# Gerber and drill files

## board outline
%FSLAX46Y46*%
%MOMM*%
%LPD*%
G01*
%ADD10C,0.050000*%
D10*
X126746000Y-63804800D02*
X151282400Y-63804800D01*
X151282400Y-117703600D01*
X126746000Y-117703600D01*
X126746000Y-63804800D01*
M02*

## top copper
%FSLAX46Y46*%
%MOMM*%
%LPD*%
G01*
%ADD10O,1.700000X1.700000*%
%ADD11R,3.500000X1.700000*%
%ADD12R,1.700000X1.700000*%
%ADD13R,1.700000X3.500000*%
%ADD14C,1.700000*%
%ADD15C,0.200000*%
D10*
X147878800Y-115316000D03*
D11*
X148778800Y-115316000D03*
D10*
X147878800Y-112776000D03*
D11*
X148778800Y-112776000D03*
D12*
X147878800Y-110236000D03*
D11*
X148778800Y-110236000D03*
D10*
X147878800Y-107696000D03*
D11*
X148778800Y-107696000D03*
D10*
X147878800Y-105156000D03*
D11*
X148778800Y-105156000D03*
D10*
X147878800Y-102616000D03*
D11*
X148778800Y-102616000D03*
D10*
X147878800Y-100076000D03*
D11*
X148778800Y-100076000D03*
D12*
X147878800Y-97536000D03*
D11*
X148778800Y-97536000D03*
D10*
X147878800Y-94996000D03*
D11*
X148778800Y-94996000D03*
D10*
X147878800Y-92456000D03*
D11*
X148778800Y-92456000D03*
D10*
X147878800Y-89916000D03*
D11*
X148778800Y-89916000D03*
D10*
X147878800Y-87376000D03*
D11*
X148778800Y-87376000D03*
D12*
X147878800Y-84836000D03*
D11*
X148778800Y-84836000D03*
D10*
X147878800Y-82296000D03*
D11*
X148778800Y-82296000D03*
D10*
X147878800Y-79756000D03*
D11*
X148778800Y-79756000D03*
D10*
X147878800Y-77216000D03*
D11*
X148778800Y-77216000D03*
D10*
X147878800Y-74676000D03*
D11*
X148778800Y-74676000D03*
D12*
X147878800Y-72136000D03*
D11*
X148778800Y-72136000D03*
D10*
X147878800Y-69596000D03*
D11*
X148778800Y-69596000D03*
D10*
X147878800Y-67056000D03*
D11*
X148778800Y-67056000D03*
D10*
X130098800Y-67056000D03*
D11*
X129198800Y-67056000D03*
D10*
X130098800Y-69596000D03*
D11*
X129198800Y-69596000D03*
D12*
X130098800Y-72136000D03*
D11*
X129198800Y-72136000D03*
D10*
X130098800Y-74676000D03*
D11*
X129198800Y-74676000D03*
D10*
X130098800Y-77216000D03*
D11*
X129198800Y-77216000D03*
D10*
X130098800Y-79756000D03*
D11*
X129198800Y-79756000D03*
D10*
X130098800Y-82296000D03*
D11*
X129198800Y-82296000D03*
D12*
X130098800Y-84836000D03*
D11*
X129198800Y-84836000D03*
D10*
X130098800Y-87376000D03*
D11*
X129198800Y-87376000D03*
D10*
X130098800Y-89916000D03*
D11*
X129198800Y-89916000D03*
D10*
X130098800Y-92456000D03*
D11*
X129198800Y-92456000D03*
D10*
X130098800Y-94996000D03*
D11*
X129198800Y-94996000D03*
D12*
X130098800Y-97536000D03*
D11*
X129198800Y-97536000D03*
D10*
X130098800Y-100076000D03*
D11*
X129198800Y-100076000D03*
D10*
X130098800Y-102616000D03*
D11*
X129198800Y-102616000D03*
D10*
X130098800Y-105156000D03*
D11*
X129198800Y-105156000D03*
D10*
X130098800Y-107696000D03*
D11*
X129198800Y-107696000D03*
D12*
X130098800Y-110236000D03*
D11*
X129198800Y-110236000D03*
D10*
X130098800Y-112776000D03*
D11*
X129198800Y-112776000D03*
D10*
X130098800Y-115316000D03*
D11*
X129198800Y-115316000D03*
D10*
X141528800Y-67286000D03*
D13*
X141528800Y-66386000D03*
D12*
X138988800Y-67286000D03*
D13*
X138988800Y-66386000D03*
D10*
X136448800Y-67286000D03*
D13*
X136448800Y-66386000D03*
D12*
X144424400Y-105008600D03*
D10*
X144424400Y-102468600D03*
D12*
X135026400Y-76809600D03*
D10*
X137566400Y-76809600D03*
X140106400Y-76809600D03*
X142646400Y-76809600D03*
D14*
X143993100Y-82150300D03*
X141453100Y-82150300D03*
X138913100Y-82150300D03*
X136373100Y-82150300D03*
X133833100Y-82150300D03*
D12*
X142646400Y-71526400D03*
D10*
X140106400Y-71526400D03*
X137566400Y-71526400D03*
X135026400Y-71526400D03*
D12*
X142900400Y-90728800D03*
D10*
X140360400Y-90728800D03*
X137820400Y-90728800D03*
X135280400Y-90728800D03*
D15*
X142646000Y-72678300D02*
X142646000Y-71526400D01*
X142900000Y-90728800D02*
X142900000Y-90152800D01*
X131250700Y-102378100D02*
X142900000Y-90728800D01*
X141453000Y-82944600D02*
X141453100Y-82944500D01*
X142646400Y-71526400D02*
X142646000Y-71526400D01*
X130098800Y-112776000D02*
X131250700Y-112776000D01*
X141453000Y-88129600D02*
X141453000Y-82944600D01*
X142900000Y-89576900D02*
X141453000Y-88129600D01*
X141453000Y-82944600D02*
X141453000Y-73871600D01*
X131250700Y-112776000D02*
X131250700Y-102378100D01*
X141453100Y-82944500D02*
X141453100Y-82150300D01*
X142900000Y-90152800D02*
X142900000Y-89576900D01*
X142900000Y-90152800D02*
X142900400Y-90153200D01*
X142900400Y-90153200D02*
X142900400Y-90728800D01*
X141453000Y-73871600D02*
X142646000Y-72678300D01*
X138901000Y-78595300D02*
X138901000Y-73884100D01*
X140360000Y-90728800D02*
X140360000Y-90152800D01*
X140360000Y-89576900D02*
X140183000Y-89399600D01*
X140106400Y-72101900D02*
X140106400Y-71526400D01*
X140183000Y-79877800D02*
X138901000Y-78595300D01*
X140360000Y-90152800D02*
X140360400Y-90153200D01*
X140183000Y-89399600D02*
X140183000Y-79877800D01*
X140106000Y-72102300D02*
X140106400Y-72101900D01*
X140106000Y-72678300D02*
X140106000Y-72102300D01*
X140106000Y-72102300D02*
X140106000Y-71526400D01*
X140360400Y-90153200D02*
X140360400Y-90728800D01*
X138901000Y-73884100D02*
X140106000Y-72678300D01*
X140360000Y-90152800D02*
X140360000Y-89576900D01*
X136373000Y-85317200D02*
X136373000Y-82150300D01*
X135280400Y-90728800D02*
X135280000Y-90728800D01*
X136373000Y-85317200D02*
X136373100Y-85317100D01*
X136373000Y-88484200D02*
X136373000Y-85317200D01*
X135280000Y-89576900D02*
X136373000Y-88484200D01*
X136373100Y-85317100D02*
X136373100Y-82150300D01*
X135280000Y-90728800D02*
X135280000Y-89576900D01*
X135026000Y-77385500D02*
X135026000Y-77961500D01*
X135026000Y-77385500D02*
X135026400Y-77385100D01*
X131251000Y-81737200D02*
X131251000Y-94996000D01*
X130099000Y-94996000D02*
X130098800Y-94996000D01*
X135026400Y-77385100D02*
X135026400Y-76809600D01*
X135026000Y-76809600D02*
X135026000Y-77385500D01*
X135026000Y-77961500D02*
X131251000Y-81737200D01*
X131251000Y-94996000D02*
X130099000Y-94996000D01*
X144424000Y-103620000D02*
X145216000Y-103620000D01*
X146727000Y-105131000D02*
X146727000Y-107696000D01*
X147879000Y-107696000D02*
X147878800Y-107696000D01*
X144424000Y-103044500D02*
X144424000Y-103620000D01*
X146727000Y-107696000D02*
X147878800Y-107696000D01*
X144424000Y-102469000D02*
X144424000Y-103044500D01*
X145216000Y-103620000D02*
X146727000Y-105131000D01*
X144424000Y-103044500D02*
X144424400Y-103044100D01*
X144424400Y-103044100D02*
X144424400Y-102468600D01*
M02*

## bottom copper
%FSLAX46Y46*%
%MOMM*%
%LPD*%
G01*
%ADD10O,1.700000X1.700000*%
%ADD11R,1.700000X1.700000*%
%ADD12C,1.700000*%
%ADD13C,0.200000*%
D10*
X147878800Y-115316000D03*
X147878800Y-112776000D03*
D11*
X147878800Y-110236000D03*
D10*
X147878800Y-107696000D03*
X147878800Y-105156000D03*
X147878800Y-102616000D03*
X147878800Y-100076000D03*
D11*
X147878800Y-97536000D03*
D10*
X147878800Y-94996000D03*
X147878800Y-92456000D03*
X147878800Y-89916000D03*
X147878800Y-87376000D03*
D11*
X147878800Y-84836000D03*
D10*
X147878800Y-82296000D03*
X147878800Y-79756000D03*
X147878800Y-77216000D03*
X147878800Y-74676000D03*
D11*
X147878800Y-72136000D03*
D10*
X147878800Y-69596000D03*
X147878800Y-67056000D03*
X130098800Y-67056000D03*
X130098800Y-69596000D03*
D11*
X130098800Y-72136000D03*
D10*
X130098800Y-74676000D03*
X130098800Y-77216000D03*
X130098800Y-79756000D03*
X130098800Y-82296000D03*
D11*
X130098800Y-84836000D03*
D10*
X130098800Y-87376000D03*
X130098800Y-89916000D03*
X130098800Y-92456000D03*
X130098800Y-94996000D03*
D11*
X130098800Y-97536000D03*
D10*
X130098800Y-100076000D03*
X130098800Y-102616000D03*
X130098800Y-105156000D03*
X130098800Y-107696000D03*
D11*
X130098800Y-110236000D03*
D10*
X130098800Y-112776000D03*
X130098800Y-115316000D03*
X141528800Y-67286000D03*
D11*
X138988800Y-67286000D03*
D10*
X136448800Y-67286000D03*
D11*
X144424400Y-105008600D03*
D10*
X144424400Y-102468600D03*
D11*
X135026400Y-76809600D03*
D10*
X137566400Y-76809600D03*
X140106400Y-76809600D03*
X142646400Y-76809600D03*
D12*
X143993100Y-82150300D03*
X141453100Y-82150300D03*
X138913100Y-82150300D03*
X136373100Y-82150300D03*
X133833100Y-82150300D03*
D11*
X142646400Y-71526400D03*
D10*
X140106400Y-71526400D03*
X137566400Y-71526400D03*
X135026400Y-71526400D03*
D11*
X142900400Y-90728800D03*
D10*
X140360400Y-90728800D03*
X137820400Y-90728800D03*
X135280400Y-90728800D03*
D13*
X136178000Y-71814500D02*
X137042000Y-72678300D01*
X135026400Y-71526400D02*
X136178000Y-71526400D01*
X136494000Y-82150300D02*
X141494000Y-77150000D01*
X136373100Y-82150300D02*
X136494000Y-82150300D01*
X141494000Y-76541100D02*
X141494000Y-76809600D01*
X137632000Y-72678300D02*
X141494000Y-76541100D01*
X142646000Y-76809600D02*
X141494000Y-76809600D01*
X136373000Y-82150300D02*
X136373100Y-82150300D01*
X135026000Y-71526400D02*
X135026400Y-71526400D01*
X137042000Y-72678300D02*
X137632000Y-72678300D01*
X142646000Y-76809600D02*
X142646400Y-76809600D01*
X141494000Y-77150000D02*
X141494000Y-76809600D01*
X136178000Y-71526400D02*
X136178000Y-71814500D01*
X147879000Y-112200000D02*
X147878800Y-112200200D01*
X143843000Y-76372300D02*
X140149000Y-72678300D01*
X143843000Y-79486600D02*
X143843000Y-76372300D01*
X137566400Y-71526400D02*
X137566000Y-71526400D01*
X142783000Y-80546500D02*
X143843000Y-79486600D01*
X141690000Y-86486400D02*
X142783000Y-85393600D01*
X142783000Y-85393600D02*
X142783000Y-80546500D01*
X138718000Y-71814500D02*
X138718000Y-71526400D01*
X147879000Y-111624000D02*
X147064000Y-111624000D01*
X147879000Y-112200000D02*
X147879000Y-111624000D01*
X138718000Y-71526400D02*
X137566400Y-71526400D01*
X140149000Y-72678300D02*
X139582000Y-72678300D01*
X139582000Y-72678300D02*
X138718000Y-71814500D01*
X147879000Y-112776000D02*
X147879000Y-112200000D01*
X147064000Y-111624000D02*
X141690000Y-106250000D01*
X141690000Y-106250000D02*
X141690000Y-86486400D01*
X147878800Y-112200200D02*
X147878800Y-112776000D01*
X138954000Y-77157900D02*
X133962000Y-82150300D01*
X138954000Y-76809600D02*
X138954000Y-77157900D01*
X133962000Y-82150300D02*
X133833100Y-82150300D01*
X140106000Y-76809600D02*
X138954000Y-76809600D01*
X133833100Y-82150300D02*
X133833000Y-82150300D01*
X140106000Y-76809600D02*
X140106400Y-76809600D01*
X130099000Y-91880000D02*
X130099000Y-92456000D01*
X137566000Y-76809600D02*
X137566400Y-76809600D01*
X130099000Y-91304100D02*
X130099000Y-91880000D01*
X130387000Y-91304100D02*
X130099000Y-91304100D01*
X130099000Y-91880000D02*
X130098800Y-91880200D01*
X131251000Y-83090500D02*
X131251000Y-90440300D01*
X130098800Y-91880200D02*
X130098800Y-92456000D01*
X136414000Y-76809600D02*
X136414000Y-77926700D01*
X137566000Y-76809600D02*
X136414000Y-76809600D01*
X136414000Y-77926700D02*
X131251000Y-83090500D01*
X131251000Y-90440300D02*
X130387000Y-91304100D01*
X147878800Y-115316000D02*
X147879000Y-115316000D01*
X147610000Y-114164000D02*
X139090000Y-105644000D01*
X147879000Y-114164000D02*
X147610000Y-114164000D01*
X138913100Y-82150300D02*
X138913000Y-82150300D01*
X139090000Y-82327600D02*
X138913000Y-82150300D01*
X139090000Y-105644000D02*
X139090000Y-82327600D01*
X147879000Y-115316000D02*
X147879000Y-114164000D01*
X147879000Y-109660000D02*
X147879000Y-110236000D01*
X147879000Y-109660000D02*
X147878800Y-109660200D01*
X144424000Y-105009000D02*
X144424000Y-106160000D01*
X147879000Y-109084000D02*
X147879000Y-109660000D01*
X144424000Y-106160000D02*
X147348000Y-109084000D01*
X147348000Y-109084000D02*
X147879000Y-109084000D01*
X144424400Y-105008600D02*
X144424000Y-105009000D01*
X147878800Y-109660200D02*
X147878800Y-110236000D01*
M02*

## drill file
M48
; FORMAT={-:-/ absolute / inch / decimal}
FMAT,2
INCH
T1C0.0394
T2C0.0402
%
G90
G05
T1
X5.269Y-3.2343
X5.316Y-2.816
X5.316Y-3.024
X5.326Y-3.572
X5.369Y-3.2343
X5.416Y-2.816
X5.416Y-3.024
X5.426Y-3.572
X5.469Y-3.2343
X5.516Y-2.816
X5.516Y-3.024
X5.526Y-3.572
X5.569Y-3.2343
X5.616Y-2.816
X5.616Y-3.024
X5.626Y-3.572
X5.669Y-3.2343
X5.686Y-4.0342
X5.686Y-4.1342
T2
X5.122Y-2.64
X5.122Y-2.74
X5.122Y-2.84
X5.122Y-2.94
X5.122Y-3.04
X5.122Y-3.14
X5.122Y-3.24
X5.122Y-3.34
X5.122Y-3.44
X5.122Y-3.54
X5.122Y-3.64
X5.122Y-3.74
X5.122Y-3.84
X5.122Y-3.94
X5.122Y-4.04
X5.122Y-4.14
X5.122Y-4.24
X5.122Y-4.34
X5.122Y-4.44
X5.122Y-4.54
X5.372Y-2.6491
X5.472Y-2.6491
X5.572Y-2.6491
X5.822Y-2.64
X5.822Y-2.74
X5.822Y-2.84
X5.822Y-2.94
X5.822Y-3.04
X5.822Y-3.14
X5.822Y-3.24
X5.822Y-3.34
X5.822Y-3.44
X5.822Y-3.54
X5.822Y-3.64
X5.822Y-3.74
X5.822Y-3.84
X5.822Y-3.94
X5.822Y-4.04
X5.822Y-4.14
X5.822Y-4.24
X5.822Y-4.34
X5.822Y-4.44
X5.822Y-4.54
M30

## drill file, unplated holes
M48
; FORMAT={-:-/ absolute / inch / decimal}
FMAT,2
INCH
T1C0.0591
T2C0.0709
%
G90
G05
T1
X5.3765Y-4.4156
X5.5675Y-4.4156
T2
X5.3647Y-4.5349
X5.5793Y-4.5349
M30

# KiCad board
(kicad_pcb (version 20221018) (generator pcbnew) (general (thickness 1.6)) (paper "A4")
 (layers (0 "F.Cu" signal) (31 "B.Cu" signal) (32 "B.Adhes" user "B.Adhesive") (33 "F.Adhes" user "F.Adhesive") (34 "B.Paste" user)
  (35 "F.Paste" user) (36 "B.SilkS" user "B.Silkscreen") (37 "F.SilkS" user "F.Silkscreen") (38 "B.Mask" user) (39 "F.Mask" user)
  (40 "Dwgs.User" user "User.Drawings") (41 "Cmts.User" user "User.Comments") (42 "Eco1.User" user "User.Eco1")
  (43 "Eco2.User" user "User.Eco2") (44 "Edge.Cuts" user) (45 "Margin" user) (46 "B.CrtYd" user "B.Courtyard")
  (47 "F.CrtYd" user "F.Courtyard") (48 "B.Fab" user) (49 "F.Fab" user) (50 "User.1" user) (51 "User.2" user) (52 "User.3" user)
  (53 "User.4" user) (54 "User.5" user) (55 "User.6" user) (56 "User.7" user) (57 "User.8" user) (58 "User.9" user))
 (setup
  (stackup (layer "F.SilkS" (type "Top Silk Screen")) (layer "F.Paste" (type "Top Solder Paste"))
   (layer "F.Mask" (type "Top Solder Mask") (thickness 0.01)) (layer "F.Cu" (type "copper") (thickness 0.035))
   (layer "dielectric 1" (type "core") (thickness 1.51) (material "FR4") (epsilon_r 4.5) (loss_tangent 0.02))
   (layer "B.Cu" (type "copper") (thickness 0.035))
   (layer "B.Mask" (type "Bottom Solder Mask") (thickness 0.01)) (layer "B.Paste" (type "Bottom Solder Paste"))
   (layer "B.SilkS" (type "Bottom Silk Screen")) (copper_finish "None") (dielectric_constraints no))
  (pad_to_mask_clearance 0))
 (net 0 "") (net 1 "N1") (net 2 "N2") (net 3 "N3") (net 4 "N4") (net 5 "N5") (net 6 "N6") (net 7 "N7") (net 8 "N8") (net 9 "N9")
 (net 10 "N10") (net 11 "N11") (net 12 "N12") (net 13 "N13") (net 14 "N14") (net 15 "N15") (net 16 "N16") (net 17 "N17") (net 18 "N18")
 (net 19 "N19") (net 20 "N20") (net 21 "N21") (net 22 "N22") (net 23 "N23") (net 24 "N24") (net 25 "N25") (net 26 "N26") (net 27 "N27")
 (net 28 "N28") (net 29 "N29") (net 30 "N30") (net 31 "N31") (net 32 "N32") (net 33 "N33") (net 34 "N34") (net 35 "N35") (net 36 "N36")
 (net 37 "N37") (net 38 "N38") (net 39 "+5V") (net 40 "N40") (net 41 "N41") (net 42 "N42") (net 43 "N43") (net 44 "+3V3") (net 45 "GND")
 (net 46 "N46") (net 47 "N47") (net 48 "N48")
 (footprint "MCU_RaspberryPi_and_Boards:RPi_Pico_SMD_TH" (layer "F.Cu") (at 138.9888 91.186 180)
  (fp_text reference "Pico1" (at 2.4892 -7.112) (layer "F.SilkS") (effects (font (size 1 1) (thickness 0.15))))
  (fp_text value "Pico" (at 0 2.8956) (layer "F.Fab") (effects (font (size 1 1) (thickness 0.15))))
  (pad "" np_thru_hole oval (at -2.725 -24 180) (size 1.8 1.8) (drill 1.8) (layers "*.Cu" "*.Mask"))
  (pad "" np_thru_hole oval (at -2.425 -20.97 180) (size 1.5 1.5) (drill 1.5) (layers "*.Cu" "*.Mask"))
  (pad "" np_thru_hole oval (at 2.425 -20.97 180) (size 1.5 1.5) (drill 1.5) (layers "*.Cu" "*.Mask"))
  (pad "" np_thru_hole oval (at 2.725 -24 180) (size 1.8 1.8) (drill 1.8) (layers "*.Cu" "*.Mask"))
  (pad "1" thru_hole oval (at -8.89 -24.13 180) (size 1.7 1.7) (drill 1.02) (layers "*.Cu" "*.Mask") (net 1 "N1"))
  (pad "1" smd rect (at -8.89 -24.13 180) (size 3.5 1.7) (drill (offset -0.9 0)) (layers "F.Cu" "F.Mask") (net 1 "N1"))
  (pad "2" thru_hole oval (at -8.89 -21.59 180) (size 1.7 1.7) (drill 1.02) (layers "*.Cu" "*.Mask") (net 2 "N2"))
  (pad "2" smd rect (at -8.89 -21.59 180) (size 3.5 1.7) (drill (offset -0.9 0)) (layers "F.Cu" "F.Mask") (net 2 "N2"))
  (pad "3" thru_hole rect (at -8.89 -19.05 180) (size 1.7 1.7) (drill 1.02) (layers "*.Cu" "*.Mask") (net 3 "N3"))
  (pad "3" smd rect (at -8.89 -19.05 180) (size 3.5 1.7) (drill (offset -0.9 0)) (layers "F.Cu" "F.Mask") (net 3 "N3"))
  (pad "4" thru_hole oval (at -8.89 -16.51 180) (size 1.7 1.7) (drill 1.02) (layers "*.Cu" "*.Mask") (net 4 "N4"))
  (pad "4" smd rect (at -8.89 -16.51 180) (size 3.5 1.7) (drill (offset -0.9 0)) (layers "F.Cu" "F.Mask") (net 4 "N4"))
  (pad "5" thru_hole oval (at -8.89 -13.97 180) (size 1.7 1.7) (drill 1.02) (layers "*.Cu" "*.Mask") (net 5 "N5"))
  (pad "5" smd rect (at -8.89 -13.97 180) (size 3.5 1.7) (drill (offset -0.9 0)) (layers "F.Cu" "F.Mask") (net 5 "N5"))
  (pad "6" thru_hole oval (at -8.89 -11.43 180) (size 1.7 1.7) (drill 1.02) (layers "*.Cu" "*.Mask") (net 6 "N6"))
  (pad "6" smd rect (at -8.89 -11.43 180) (size 3.5 1.7) (drill (offset -0.9 0)) (layers "F.Cu" "F.Mask") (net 6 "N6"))
  (pad "7" thru_hole oval (at -8.89 -8.89 180) (size 1.7 1.7) (drill 1.02) (layers "*.Cu" "*.Mask") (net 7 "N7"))
  (pad "7" smd rect (at -8.89 -8.89 180) (size 3.5 1.7) (drill (offset -0.9 0)) (layers "F.Cu" "F.Mask") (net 7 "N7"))
  (pad "8" thru_hole rect (at -8.89 -6.35 180) (size 1.7 1.7) (drill 1.02) (layers "*.Cu" "*.Mask") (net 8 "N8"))
  (pad "8" smd rect (at -8.89 -6.35 180) (size 3.5 1.7) (drill (offset -0.9 0)) (layers "F.Cu" "F.Mask") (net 8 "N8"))
  (pad "9" thru_hole oval (at -8.89 -3.81 180) (size 1.7 1.7) (drill 1.02) (layers "*.Cu" "*.Mask") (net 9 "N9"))
  (pad "9" smd rect (at -8.89 -3.81 180) (size 3.5 1.7) (drill (offset -0.9 0)) (layers "F.Cu" "F.Mask") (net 9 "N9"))
  (pad "10" thru_hole oval (at -8.89 -1.27 180) (size 1.7 1.7) (drill 1.02) (layers "*.Cu" "*.Mask") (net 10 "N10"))
  (pad "10" smd rect (at -8.89 -1.27 180) (size 3.5 1.7) (drill (offset -0.9 0)) (layers "F.Cu" "F.Mask") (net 10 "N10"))
  (pad "11" thru_hole oval (at -8.89 1.27 180) (size 1.7 1.7) (drill 1.02) (layers "*.Cu" "*.Mask") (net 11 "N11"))
  (pad "11" smd rect (at -8.89 1.27 180) (size 3.5 1.7) (drill (offset -0.9 0)) (layers "F.Cu" "F.Mask") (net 11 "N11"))
  (pad "12" thru_hole oval (at -8.89 3.81 180) (size 1.7 1.7) (drill 1.02) (layers "*.Cu" "*.Mask") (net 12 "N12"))
  (pad "12" smd rect (at -8.89 3.81 180) (size 3.5 1.7) (drill (offset -0.9 0)) (layers "F.Cu" "F.Mask") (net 12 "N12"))
  (pad "13" thru_hole rect (at -8.89 6.35 180) (size 1.7 1.7) (drill 1.02) (layers "*.Cu" "*.Mask") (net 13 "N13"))
  (pad "13" smd rect (at -8.89 6.35 180) (size 3.5 1.7) (drill (offset -0.9 0)) (layers "F.Cu" "F.Mask") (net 13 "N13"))
  (pad "14" thru_hole oval (at -8.89 8.89 180) (size 1.7 1.7) (drill 1.02) (layers "*.Cu" "*.Mask") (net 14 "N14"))
  (pad "14" smd rect (at -8.89 8.89 180) (size 3.5 1.7) (drill (offset -0.9 0)) (layers "F.Cu" "F.Mask") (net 14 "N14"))
  (pad "15" thru_hole oval (at -8.89 11.43 180) (size 1.7 1.7) (drill 1.02) (layers "*.Cu" "*.Mask") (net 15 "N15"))
  (pad "15" smd rect (at -8.89 11.43 180) (size 3.5 1.7) (drill (offset -0.9 0)) (layers "F.Cu" "F.Mask") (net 15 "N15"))
  (pad "16" thru_hole oval (at -8.89 13.97 180) (size 1.7 1.7) (drill 1.02) (layers "*.Cu" "*.Mask") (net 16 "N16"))
  (pad "16" smd rect (at -8.89 13.97 180) (size 3.5 1.7) (drill (offset -0.9 0)) (layers "F.Cu" "F.Mask") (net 16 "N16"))
  (pad "17" thru_hole oval (at -8.89 16.51 180) (size 1.7 1.7) (drill 1.02) (layers "*.Cu" "*.Mask") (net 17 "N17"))
  (pad "17" smd rect (at -8.89 16.51 180) (size 3.5 1.7) (drill (offset -0.9 0)) (layers "F.Cu" "F.Mask") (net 17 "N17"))
  (pad "18" thru_hole rect (at -8.89 19.05 180) (size 1.7 1.7) (drill 1.02) (layers "*.Cu" "*.Mask") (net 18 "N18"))
  (pad "18" smd rect (at -8.89 19.05 180) (size 3.5 1.7) (drill (offset -0.9 0)) (layers "F.Cu" "F.Mask") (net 18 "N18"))
  (pad "19" thru_hole oval (at -8.89 21.59 180) (size 1.7 1.7) (drill 1.02) (layers "*.Cu" "*.Mask") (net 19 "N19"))
  (pad "19" smd rect (at -8.89 21.59 180) (size 3.5 1.7) (drill (offset -0.9 0)) (layers "F.Cu" "F.Mask") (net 19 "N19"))
  (pad "20" thru_hole oval (at -8.89 24.13 180) (size 1.7 1.7) (drill 1.02) (layers "*.Cu" "*.Mask") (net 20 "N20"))
  (pad "20" smd rect (at -8.89 24.13 180) (size 3.5 1.7) (drill (offset -0.9 0)) (layers "F.Cu" "F.Mask") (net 20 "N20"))
  (pad "21" thru_hole oval (at 8.89 24.13 180) (size 1.7 1.7) (drill 1.02) (layers "*.Cu" "*.Mask") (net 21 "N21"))
  (pad "21" smd rect (at 8.89 24.13 180) (size 3.5 1.7) (drill (offset 0.9 0)) (layers "F.Cu" "F.Mask") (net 21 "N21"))
  (pad "22" thru_hole oval (at 8.89 21.59 180) (size 1.7 1.7) (drill 1.02) (layers "*.Cu" "*.Mask") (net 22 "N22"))
  (pad "22" smd rect (at 8.89 21.59 180) (size 3.5 1.7) (drill (offset 0.9 0)) (layers "F.Cu" "F.Mask") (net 22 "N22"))
  (pad "23" thru_hole rect (at 8.89 19.05 180) (size 1.7 1.7) (drill 1.02) (layers "*.Cu" "*.Mask") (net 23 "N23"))
  (pad "23" smd rect (at 8.89 19.05 180) (size 3.5 1.7) (drill (offset 0.9 0)) (layers "F.Cu" "F.Mask") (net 23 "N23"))
  (pad "24" thru_hole oval (at 8.89 16.51 180) (size 1.7 1.7) (drill 1.02) (layers "*.Cu" "*.Mask") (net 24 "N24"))
  (pad "24" smd rect (at 8.89 16.51 180) (size 3.5 1.7) (drill (offset 0.9 0)) (layers "F.Cu" "F.Mask") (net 24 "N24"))
  (pad "25" thru_hole oval (at 8.89 13.97 180) (size 1.7 1.7) (drill 1.02) (layers "*.Cu" "*.Mask") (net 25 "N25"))
  (pad "25" smd rect (at 8.89 13.97 180) (size 3.5 1.7) (drill (offset 0.9 0)) (layers "F.Cu" "F.Mask") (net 25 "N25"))
  (pad "26" thru_hole oval (at 8.89 11.43 180) (size 1.7 1.7) (drill 1.02) (layers "*.Cu" "*.Mask") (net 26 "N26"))
  (pad "26" smd rect (at 8.89 11.43 180) (size 3.5 1.7) (drill (offset 0.9 0)) (layers "F.Cu" "F.Mask") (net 26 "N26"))
  (pad "27" thru_hole oval (at 8.89 8.89 180) (size 1.7 1.7) (drill 1.02) (layers "*.Cu" "*.Mask") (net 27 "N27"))
  (pad "27" smd rect (at 8.89 8.89 180) (size 3.5 1.7) (drill (offset 0.9 0)) (layers "F.Cu" "F.Mask") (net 27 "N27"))
  (pad "28" thru_hole rect (at 8.89 6.35 180) (size 1.7 1.7) (drill 1.02) (layers "*.Cu" "*.Mask") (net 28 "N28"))
  (pad "28" smd rect (at 8.89 6.35 180) (size 3.5 1.7) (drill (offset 0.9 0)) (layers "F.Cu" "F.Mask") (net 28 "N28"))
  (pad "29" thru_hole oval (at 8.89 3.81 180) (size 1.7 1.7) (drill 1.02) (layers "*.Cu" "*.Mask") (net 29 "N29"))
  (pad "29" smd rect (at 8.89 3.81 180) (size 3.5 1.7) (drill (offset 0.9 0)) (layers "F.Cu" "F.Mask") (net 29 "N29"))
  (pad "30" thru_hole oval (at 8.89 1.27 180) (size 1.7 1.7) (drill 1.02) (layers "*.Cu" "*.Mask") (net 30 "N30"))
  (pad "30" smd rect (at 8.89 1.27 180) (size 3.5 1.7) (drill (offset 0.9 0)) (layers "F.Cu" "F.Mask") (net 30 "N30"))
  (pad "31" thru_hole oval (at 8.89 -1.27 180) (size 1.7 1.7) (drill 1.02) (layers "*.Cu" "*.Mask") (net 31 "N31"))
  (pad "31" smd rect (at 8.89 -1.27 180) (size 3.5 1.7) (drill (offset 0.9 0)) (layers "F.Cu" "F.Mask") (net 31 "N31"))
  (pad "32" thru_hole oval (at 8.89 -3.81 180) (size 1.7 1.7) (drill 1.02) (layers "*.Cu" "*.Mask") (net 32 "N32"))
  (pad "32" smd rect (at 8.89 -3.81 180) (size 3.5 1.7) (drill (offset 0.9 0)) (layers "F.Cu" "F.Mask") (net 32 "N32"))
  (pad "33" thru_hole rect (at 8.89 -6.35 180) (size 1.7 1.7) (drill 1.02) (layers "*.Cu" "*.Mask") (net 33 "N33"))
  (pad "33" smd rect (at 8.89 -6.35 180) (size 3.5 1.7) (drill (offset 0.9 0)) (layers "F.Cu" "F.Mask") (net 33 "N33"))
  (pad "34" thru_hole oval (at 8.89 -8.89 180) (size 1.7 1.7) (drill 1.02) (layers "*.Cu" "*.Mask") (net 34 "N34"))
  (pad "34" smd rect (at 8.89 -8.89 180) (size 3.5 1.7) (drill (offset 0.9 0)) (layers "F.Cu" "F.Mask") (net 34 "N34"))
  (pad "35" thru_hole oval (at 8.89 -11.43 180) (size 1.7 1.7) (drill 1.02) (layers "*.Cu" "*.Mask") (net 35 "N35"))
  (pad "35" smd rect (at 8.89 -11.43 180) (size 3.5 1.7) (drill (offset 0.9 0)) (layers "F.Cu" "F.Mask") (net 35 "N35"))
  (pad "36" thru_hole oval (at 8.89 -13.97 180) (size 1.7 1.7) (drill 1.02) (layers "*.Cu" "*.Mask") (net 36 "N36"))
  (pad "36" smd rect (at 8.89 -13.97 180) (size 3.5 1.7) (drill (offset 0.9 0)) (layers "F.Cu" "F.Mask") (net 36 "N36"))
  (pad "37" thru_hole oval (at 8.89 -16.51 180) (size 1.7 1.7) (drill 1.02) (layers "*.Cu" "*.Mask") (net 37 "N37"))
  (pad "37" smd rect (at 8.89 -16.51 180) (size 3.5 1.7) (drill (offset 0.9 0)) (layers "F.Cu" "F.Mask") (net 37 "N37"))
  (pad "38" thru_hole rect (at 8.89 -19.05 180) (size 1.7 1.7) (drill 1.02) (layers "*.Cu" "*.Mask") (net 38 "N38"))
  (pad "38" smd rect (at 8.89 -19.05 180) (size 3.5 1.7) (drill (offset 0.9 0)) (layers "F.Cu" "F.Mask") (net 38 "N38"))
  (pad "39" thru_hole oval (at 8.89 -21.59 180) (size 1.7 1.7) (drill 1.02) (layers "*.Cu" "*.Mask") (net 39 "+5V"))
  (pad "39" smd rect (at 8.89 -21.59 180) (size 3.5 1.7) (drill (offset 0.9 0)) (layers "F.Cu" "F.Mask") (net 39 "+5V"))
  (pad "40" thru_hole oval (at 8.89 -24.13 180) (size 1.7 1.7) (drill 1.02) (layers "*.Cu" "*.Mask") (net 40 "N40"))
  (pad "40" smd rect (at 8.89 -24.13 180) (size 3.5 1.7) (drill (offset 0.9 0)) (layers "F.Cu" "F.Mask") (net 40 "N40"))
  (pad "41" thru_hole oval (at -2.54 23.9 180) (size 1.7 1.7) (drill 1.02) (layers "*.Cu" "*.Mask") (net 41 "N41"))
  (pad "41" smd rect (at -2.54 23.9 270) (size 3.5 1.7) (drill (offset -0.9 0)) (layers "F.Cu" "F.Mask") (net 41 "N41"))
  (pad "42" thru_hole rect (at 0 23.9 180) (size 1.7 1.7) (drill 1.02) (layers "*.Cu" "*.Mask") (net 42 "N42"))
  (pad "42" smd rect (at 0 23.9 270) (size 3.5 1.7) (drill (offset -0.9 0)) (layers "F.Cu" "F.Mask") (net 42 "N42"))
  (pad "43" thru_hole oval (at 2.54 23.9 180) (size 1.7 1.7) (drill 1.02) (layers "*.Cu" "*.Mask") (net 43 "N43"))
  (pad "43" smd rect (at 2.54 23.9 270) (size 3.5 1.7) (drill (offset -0.9 0)) (layers "F.Cu" "F.Mask") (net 43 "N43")))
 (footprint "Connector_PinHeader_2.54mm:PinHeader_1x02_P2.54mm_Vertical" (layer "B.Cu") (at 144.4244 105.0086)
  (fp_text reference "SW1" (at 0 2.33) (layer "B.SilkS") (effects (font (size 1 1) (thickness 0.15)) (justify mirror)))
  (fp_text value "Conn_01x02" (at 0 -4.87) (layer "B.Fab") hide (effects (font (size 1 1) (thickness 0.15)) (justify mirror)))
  (pad "1" thru_hole rect (at 0 0) (size 1.7 1.7) (drill 1) (layers "*.Cu" "*.Mask") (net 3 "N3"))
  (pad "2" thru_hole oval (at 0 -2.54) (size 1.7 1.7) (drill 1) (layers "*.Cu" "*.Mask") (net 4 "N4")))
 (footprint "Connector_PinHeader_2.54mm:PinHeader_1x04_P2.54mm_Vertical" (layer "B.Cu") (at 135.0264 76.8096 -90)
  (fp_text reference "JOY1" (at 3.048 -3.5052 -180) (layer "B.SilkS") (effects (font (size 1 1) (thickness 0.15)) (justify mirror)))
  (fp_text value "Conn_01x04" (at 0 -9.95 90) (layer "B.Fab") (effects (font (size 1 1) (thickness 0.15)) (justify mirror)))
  (pad "1" thru_hole rect (at 0 0 270) (size 1.7 1.7) (drill 1) (layers "*.Cu" "*.Mask") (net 32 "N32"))
  (pad "2" thru_hole oval (at 0 -2.54 270) (size 1.7 1.7) (drill 1) (layers "*.Cu" "*.Mask") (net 31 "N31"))
  (pad "3" thru_hole oval (at 0 -5.08 270) (size 1.7 1.7) (drill 1) (layers "*.Cu" "*.Mask") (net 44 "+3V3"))
  (pad "4" thru_hole oval (at 0 -7.62 270) (size 1.7 1.7) (drill 1) (layers "*.Cu" "*.Mask") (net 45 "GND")))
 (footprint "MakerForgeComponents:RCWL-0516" (layer "B.Cu") (at 130.0231 79.6103)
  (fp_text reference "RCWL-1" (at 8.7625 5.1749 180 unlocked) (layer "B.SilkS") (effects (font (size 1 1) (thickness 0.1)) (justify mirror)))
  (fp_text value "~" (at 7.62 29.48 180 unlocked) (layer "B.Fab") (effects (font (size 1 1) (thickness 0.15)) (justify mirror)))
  (pad "1" thru_hole circle (at 13.97 2.54) (size 1.7 1.7) (drill 1) (layers "*.Cu" "*.Mask") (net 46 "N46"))
  (pad "2" thru_hole circle (at 11.43 2.54) (size 1.7 1.7) (drill 1) (layers "*.Cu" "*.Mask") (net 39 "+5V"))
  (pad "3" thru_hole circle (at 8.89 2.54) (size 1.7 1.7) (drill 1) (layers "*.Cu" "*.Mask") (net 1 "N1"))
  (pad "4" thru_hole circle (at 6.35 2.54) (size 1.7 1.7) (drill 1) (layers "*.Cu" "*.Mask") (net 45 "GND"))
  (pad "5" thru_hole circle (at 3.81 2.54) (size 1.7 1.7) (drill 1) (layers "*.Cu" "*.Mask") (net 44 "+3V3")))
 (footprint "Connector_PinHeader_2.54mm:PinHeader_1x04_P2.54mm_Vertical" (layer "B.Cu") (at 142.6464 71.5264 90)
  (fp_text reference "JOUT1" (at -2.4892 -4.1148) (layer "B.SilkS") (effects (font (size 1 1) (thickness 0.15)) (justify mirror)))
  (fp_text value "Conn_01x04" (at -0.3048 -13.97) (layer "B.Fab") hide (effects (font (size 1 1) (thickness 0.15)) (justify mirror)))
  (pad "1" thru_hole rect (at 0 0 90) (size 1.7 1.7) (drill 1) (layers "*.Cu" "*.Mask") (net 39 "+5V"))
  (pad "2" thru_hole oval (at 0 -2.54 90) (size 1.7 1.7) (drill 1) (layers "*.Cu" "*.Mask") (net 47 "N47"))
  (pad "3" thru_hole oval (at 0 -5.08 90) (size 1.7 1.7) (drill 1) (layers "*.Cu" "*.Mask") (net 2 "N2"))
  (pad "4" thru_hole oval (at 0 -7.62 90) (size 1.7 1.7) (drill 1) (layers "*.Cu" "*.Mask") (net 45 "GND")))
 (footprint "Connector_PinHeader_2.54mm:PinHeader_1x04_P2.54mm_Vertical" (layer "B.Cu") (at 142.9004 90.7288 90)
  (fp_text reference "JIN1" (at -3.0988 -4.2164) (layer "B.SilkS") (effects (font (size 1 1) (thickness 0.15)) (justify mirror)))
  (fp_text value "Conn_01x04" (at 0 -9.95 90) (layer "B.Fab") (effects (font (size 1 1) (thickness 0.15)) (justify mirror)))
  (pad "1" thru_hole rect (at 0 0 90) (size 1.7 1.7) (drill 1) (layers "*.Cu" "*.Mask") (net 39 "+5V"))
  (pad "2" thru_hole oval (at 0 -2.54 90) (size 1.7 1.7) (drill 1) (layers "*.Cu" "*.Mask") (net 47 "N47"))
  (pad "3" thru_hole oval (at 0 -5.08 90) (size 1.7 1.7) (drill 1) (layers "*.Cu" "*.Mask") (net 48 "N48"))
  (pad "4" thru_hole oval (at 0 -7.62 90) (size 1.7 1.7) (drill 1) (layers "*.Cu" "*.Mask") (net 45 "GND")))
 (gr_rect (start 126.746 63.8048) (end 151.2824 117.7036) (stroke (width 0.05) (type default)) (fill none) (layer "Edge.Cuts"))
 (segment (start 142.646 72.6783) (end 142.646 71.5264) (width 0.2) (layer "F.Cu") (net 39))
 (segment (start 142.9 90.7288) (end 142.9 90.1528) (width 0.2) (layer "F.Cu") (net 39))
 (segment (start 131.2507 102.3781) (end 142.9 90.7288) (width 0.2) (layer "F.Cu") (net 39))
 (segment (start 141.453 82.9446) (end 141.4531 82.9445) (width 0.2) (layer "F.Cu") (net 39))
 (segment (start 142.6464 71.5264) (end 142.646 71.5264) (width 0.2) (layer "F.Cu") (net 39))
 (segment (start 130.0988 112.776) (end 131.2507 112.776) (width 0.2) (layer "F.Cu") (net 39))
 (segment (start 141.453 88.1296) (end 141.453 82.9446) (width 0.2) (layer "F.Cu") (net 39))
 (segment (start 142.9 89.5769) (end 141.453 88.1296) (width 0.2) (layer "F.Cu") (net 39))
 (segment (start 141.453 82.9446) (end 141.453 73.8716) (width 0.2) (layer "F.Cu") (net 39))
 (segment (start 131.2507 112.776) (end 131.2507 102.3781) (width 0.2) (layer "F.Cu") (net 39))
 (segment (start 141.4531 82.9445) (end 141.4531 82.1503) (width 0.2) (layer "F.Cu") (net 39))
 (segment (start 142.9 90.1528) (end 142.9 89.5769) (width 0.2) (layer "F.Cu") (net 39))
 (segment (start 142.9 90.1528) (end 142.9004 90.1532) (width 0.2) (layer "F.Cu") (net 39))
 (segment (start 142.9004 90.1532) (end 142.9004 90.7288) (width 0.2) (layer "F.Cu") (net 39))
 (segment (start 141.453 73.8716) (end 142.646 72.6783) (width 0.2) (layer "F.Cu") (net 39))
 (segment (start 138.901 78.5953) (end 138.901 73.8841) (width 0.2) (layer "F.Cu") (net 47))
 (segment (start 140.36 90.7288) (end 140.36 90.1528) (width 0.2) (layer "F.Cu") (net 47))
 (segment (start 140.36 89.5769) (end 140.183 89.3996) (width 0.2) (layer "F.Cu") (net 47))
 (segment (start 140.1064 72.1019) (end 140.1064 71.5264) (width 0.2) (layer "F.Cu") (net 47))
 (segment (start 140.183 79.8778) (end 138.901 78.5953) (width 0.2) (layer "F.Cu") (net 47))
 (segment (start 140.36 90.1528) (end 140.3604 90.1532) (width 0.2) (layer "F.Cu") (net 47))
 (segment (start 140.183 89.3996) (end 140.183 79.8778) (width 0.2) (layer "F.Cu") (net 47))
 (segment (start 140.106 72.1023) (end 140.1064 72.1019) (width 0.2) (layer "F.Cu") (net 47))
 (segment (start 140.106 72.6783) (end 140.106 72.1023) (width 0.2) (layer "F.Cu") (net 47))
 (segment (start 140.106 72.1023) (end 140.106 71.5264) (width 0.2) (layer "F.Cu") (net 47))
 (segment (start 140.3604 90.1532) (end 140.3604 90.7288) (width 0.2) (layer "F.Cu") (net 47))
 (segment (start 138.901 73.8841) (end 140.106 72.6783) (width 0.2) (layer "F.Cu") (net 47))
 (segment (start 140.36 90.1528) (end 140.36 89.5769) (width 0.2) (layer "F.Cu") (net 47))
 (segment (start 136.373 85.3172) (end 136.373 82.1503) (width 0.2) (layer "F.Cu") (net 45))
 (segment (start 135.2804 90.7288) (end 135.28 90.7288) (width 0.2) (layer "F.Cu") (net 45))
 (segment (start 136.373 85.3172) (end 136.3731 85.3171) (width 0.2) (layer "F.Cu") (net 45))
 (segment (start 136.373 88.4842) (end 136.373 85.3172) (width 0.2) (layer "F.Cu") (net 45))
 (segment (start 135.28 89.5769) (end 136.373 88.4842) (width 0.2) (layer "F.Cu") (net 45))
 (segment (start 136.3731 85.3171) (end 136.3731 82.1503) (width 0.2) (layer "F.Cu") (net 45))
 (segment (start 135.28 90.7288) (end 135.28 89.5769) (width 0.2) (layer "F.Cu") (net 45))
 (segment (start 136.178 71.8145) (end 137.042 72.6783) (width 0.2) (layer "B.Cu") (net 45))
 (segment (start 135.0264 71.5264) (end 136.178 71.5264) (width 0.2) (layer "B.Cu") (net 45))
 (segment (start 136.494 82.1503) (end 141.494 77.15) (width 0.2) (layer "B.Cu") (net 45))
 (segment (start 136.3731 82.1503) (end 136.494 82.1503) (width 0.2) (layer "B.Cu") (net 45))
 (segment (start 141.494 76.5411) (end 141.494 76.8096) (width 0.2) (layer "B.Cu") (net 45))
 (segment (start 137.632 72.6783) (end 141.494 76.5411) (width 0.2) (layer "B.Cu") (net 45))
 (segment (start 142.646 76.8096) (end 141.494 76.8096) (width 0.2) (layer "B.Cu") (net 45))
 (segment (start 136.373 82.1503) (end 136.3731 82.1503) (width 0.2) (layer "B.Cu") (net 45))
 (segment (start 135.026 71.5264) (end 135.0264 71.5264) (width 0.2) (layer "B.Cu") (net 45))
 (segment (start 137.042 72.6783) (end 137.632 72.6783) (width 0.2) (layer "B.Cu") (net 45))
 (segment (start 142.646 76.8096) (end 142.6464 76.8096) (width 0.2) (layer "B.Cu") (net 45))
 (segment (start 141.494 77.15) (end 141.494 76.8096) (width 0.2) (layer "B.Cu") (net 45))
 (segment (start 136.178 71.5264) (end 136.178 71.8145) (width 0.2) (layer "B.Cu") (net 45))
 (segment (start 147.879 112.2) (end 147.8788 112.2002) (width 0.2) (layer "B.Cu") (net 2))
 (segment (start 143.843 76.3723) (end 140.149 72.6783) (width 0.2) (layer "B.Cu") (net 2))
 (segment (start 143.843 79.4866) (end 143.843 76.3723) (width 0.2) (layer "B.Cu") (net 2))
 (segment (start 137.5664 71.5264) (end 137.566 71.5264) (width 0.2) (layer "B.Cu") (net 2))
 (segment (start 142.783 80.5465) (end 143.843 79.4866) (width 0.2) (layer "B.Cu") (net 2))
 (segment (start 141.69 86.4864) (end 142.783 85.3936) (width 0.2) (layer "B.Cu") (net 2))
 (segment (start 142.783 85.3936) (end 142.783 80.5465) (width 0.2) (layer "B.Cu") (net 2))
 (segment (start 138.718 71.8145) (end 138.718 71.5264) (width 0.2) (layer "B.Cu") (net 2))
 (segment (start 147.879 111.624) (end 147.064 111.624) (width 0.2) (layer "B.Cu") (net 2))
 (segment (start 147.879 112.2) (end 147.879 111.624) (width 0.2) (layer "B.Cu") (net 2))
 (segment (start 138.718 71.5264) (end 137.5664 71.5264) (width 0.2) (layer "B.Cu") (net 2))
 (segment (start 140.149 72.6783) (end 139.582 72.6783) (width 0.2) (layer "B.Cu") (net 2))
 (segment (start 139.582 72.6783) (end 138.718 71.8145) (width 0.2) (layer "B.Cu") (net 2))
 (segment (start 147.879 112.776) (end 147.879 112.2) (width 0.2) (layer "B.Cu") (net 2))
 (segment (start 147.064 111.624) (end 141.69 106.25) (width 0.2) (layer "B.Cu") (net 2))
 (segment (start 141.69 106.25) (end 141.69 86.4864) (width 0.2) (layer "B.Cu") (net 2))
 (segment (start 147.8788 112.2002) (end 147.8788 112.776) (width 0.2) (layer "B.Cu") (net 2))
 (segment (start 138.954 77.1579) (end 133.962 82.1503) (width 0.2) (layer "B.Cu") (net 44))
 (segment (start 138.954 76.8096) (end 138.954 77.1579) (width 0.2) (layer "B.Cu") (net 44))
 (segment (start 133.962 82.1503) (end 133.8331 82.1503) (width 0.2) (layer "B.Cu") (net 44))
 (segment (start 140.106 76.8096) (end 138.954 76.8096) (width 0.2) (layer "B.Cu") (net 44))
 (segment (start 133.8331 82.1503) (end 133.833 82.1503) (width 0.2) (layer "B.Cu") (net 44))
 (segment (start 140.106 76.8096) (end 140.1064 76.8096) (width 0.2) (layer "B.Cu") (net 44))
 (segment (start 135.026 77.3855) (end 135.026 77.9615) (width 0.2) (layer "F.Cu") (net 32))
 (segment (start 135.026 77.3855) (end 135.0264 77.3851) (width 0.2) (layer "F.Cu") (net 32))
 (segment (start 131.251 81.7372) (end 131.251 94.996) (width 0.2) (layer "F.Cu") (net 32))
 (segment (start 130.099 94.996) (end 130.0988 94.996) (width 0.2) (layer "F.Cu") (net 32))
 (segment (start 135.0264 77.3851) (end 135.0264 76.8096) (width 0.2) (layer "F.Cu") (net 32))
 (segment (start 135.026 76.8096) (end 135.026 77.3855) (width 0.2) (layer "F.Cu") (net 32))
 (segment (start 135.026 77.9615) (end 131.251 81.7372) (width 0.2) (layer "F.Cu") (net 32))
 (segment (start 131.251 94.996) (end 130.099 94.996) (width 0.2) (layer "F.Cu") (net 32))
 (segment (start 130.099 91.88) (end 130.099 92.456) (width 0.2) (layer "B.Cu") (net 31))
 (segment (start 137.566 76.8096) (end 137.5664 76.8096) (width 0.2) (layer "B.Cu") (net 31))
 (segment (start 130.099 91.3041) (end 130.099 91.88) (width 0.2) (layer "B.Cu") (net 31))
 (segment (start 130.387 91.3041) (end 130.099 91.3041) (width 0.2) (layer "B.Cu") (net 31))
 (segment (start 130.099 91.88) (end 130.0988 91.8802) (width 0.2) (layer "B.Cu") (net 31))
 (segment (start 131.251 83.0905) (end 131.251 90.4403) (width 0.2) (layer "B.Cu") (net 31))
 (segment (start 130.0988 91.8802) (end 130.0988 92.456) (width 0.2) (layer "B.Cu") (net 31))
 (segment (start 136.414 76.8096) (end 136.414 77.9267) (width 0.2) (layer "B.Cu") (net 31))
 (segment (start 137.566 76.8096) (end 136.414 76.8096) (width 0.2) (layer "B.Cu") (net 31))
 (segment (start 136.414 77.9267) (end 131.251 83.0905) (width 0.2) (layer "B.Cu") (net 31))
 (segment (start 131.251 90.4403) (end 130.387 91.3041) (width 0.2) (layer "B.Cu") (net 31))
 (segment (start 147.8788 115.316) (end 147.879 115.316) (width 0.2) (layer "B.Cu") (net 1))
 (segment (start 147.61 114.164) (end 139.09 105.644) (width 0.2) (layer "B.Cu") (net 1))
 (segment (start 147.879 114.164) (end 147.61 114.164) (width 0.2) (layer "B.Cu") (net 1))
 (segment (start 138.9131 82.1503) (end 138.913 82.1503) (width 0.2) (layer "B.Cu") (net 1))
 (segment (start 139.09 82.3276) (end 138.913 82.1503) (width 0.2) (layer "B.Cu") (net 1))
 (segment (start 139.09 105.644) (end 139.09 82.3276) (width 0.2) (layer "B.Cu") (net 1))
 (segment (start 147.879 115.316) (end 147.879 114.164) (width 0.2) (layer "B.Cu") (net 1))
 (segment (start 147.879 109.66) (end 147.879 110.236) (width 0.2) (layer "B.Cu") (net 3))
 (segment (start 147.879 109.66) (end 147.8788 109.6602) (width 0.2) (layer "B.Cu") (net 3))
 (segment (start 144.424 105.009) (end 144.424 106.16) (width 0.2) (layer "B.Cu") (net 3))
 (segment (start 147.879 109.084) (end 147.879 109.66) (width 0.2) (layer "B.Cu") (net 3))
 (segment (start 144.424 106.16) (end 147.348 109.084) (width 0.2) (layer "B.Cu") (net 3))
 (segment (start 147.348 109.084) (end 147.879 109.084) (width 0.2) (layer "B.Cu") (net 3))
 (segment (start 144.4244 105.0086) (end 144.424 105.009) (width 0.2) (layer "B.Cu") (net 3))
 (segment (start 147.8788 109.6602) (end 147.8788 110.236) (width 0.2) (layer "B.Cu") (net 3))
 (segment (start 144.424 103.62) (end 145.216 103.62) (width 0.2) (layer "F.Cu") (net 4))
 (segment (start 146.727 105.131) (end 146.727 107.696) (width 0.2) (layer "F.Cu") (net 4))
 (segment (start 147.879 107.696) (end 147.8788 107.696) (width 0.2) (layer "F.Cu") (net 4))
 (segment (start 144.424 103.0445) (end 144.424 103.62) (width 0.2) (layer "F.Cu") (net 4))
 (segment (start 146.727 107.696) (end 147.8788 107.696) (width 0.2) (layer "F.Cu") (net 4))
 (segment (start 144.424 102.469) (end 144.424 103.0445) (width 0.2) (layer "F.Cu") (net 4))
 (segment (start 145.216 103.62) (end 146.727 105.131) (width 0.2) (layer "F.Cu") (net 4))
 (segment (start 144.424 103.0445) (end 144.4244 103.0441) (width 0.2) (layer "F.Cu") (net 4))
 (segment (start 144.4244 103.0441) (end 144.4244 102.4686) (width 0.2) (layer "F.Cu") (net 4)))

